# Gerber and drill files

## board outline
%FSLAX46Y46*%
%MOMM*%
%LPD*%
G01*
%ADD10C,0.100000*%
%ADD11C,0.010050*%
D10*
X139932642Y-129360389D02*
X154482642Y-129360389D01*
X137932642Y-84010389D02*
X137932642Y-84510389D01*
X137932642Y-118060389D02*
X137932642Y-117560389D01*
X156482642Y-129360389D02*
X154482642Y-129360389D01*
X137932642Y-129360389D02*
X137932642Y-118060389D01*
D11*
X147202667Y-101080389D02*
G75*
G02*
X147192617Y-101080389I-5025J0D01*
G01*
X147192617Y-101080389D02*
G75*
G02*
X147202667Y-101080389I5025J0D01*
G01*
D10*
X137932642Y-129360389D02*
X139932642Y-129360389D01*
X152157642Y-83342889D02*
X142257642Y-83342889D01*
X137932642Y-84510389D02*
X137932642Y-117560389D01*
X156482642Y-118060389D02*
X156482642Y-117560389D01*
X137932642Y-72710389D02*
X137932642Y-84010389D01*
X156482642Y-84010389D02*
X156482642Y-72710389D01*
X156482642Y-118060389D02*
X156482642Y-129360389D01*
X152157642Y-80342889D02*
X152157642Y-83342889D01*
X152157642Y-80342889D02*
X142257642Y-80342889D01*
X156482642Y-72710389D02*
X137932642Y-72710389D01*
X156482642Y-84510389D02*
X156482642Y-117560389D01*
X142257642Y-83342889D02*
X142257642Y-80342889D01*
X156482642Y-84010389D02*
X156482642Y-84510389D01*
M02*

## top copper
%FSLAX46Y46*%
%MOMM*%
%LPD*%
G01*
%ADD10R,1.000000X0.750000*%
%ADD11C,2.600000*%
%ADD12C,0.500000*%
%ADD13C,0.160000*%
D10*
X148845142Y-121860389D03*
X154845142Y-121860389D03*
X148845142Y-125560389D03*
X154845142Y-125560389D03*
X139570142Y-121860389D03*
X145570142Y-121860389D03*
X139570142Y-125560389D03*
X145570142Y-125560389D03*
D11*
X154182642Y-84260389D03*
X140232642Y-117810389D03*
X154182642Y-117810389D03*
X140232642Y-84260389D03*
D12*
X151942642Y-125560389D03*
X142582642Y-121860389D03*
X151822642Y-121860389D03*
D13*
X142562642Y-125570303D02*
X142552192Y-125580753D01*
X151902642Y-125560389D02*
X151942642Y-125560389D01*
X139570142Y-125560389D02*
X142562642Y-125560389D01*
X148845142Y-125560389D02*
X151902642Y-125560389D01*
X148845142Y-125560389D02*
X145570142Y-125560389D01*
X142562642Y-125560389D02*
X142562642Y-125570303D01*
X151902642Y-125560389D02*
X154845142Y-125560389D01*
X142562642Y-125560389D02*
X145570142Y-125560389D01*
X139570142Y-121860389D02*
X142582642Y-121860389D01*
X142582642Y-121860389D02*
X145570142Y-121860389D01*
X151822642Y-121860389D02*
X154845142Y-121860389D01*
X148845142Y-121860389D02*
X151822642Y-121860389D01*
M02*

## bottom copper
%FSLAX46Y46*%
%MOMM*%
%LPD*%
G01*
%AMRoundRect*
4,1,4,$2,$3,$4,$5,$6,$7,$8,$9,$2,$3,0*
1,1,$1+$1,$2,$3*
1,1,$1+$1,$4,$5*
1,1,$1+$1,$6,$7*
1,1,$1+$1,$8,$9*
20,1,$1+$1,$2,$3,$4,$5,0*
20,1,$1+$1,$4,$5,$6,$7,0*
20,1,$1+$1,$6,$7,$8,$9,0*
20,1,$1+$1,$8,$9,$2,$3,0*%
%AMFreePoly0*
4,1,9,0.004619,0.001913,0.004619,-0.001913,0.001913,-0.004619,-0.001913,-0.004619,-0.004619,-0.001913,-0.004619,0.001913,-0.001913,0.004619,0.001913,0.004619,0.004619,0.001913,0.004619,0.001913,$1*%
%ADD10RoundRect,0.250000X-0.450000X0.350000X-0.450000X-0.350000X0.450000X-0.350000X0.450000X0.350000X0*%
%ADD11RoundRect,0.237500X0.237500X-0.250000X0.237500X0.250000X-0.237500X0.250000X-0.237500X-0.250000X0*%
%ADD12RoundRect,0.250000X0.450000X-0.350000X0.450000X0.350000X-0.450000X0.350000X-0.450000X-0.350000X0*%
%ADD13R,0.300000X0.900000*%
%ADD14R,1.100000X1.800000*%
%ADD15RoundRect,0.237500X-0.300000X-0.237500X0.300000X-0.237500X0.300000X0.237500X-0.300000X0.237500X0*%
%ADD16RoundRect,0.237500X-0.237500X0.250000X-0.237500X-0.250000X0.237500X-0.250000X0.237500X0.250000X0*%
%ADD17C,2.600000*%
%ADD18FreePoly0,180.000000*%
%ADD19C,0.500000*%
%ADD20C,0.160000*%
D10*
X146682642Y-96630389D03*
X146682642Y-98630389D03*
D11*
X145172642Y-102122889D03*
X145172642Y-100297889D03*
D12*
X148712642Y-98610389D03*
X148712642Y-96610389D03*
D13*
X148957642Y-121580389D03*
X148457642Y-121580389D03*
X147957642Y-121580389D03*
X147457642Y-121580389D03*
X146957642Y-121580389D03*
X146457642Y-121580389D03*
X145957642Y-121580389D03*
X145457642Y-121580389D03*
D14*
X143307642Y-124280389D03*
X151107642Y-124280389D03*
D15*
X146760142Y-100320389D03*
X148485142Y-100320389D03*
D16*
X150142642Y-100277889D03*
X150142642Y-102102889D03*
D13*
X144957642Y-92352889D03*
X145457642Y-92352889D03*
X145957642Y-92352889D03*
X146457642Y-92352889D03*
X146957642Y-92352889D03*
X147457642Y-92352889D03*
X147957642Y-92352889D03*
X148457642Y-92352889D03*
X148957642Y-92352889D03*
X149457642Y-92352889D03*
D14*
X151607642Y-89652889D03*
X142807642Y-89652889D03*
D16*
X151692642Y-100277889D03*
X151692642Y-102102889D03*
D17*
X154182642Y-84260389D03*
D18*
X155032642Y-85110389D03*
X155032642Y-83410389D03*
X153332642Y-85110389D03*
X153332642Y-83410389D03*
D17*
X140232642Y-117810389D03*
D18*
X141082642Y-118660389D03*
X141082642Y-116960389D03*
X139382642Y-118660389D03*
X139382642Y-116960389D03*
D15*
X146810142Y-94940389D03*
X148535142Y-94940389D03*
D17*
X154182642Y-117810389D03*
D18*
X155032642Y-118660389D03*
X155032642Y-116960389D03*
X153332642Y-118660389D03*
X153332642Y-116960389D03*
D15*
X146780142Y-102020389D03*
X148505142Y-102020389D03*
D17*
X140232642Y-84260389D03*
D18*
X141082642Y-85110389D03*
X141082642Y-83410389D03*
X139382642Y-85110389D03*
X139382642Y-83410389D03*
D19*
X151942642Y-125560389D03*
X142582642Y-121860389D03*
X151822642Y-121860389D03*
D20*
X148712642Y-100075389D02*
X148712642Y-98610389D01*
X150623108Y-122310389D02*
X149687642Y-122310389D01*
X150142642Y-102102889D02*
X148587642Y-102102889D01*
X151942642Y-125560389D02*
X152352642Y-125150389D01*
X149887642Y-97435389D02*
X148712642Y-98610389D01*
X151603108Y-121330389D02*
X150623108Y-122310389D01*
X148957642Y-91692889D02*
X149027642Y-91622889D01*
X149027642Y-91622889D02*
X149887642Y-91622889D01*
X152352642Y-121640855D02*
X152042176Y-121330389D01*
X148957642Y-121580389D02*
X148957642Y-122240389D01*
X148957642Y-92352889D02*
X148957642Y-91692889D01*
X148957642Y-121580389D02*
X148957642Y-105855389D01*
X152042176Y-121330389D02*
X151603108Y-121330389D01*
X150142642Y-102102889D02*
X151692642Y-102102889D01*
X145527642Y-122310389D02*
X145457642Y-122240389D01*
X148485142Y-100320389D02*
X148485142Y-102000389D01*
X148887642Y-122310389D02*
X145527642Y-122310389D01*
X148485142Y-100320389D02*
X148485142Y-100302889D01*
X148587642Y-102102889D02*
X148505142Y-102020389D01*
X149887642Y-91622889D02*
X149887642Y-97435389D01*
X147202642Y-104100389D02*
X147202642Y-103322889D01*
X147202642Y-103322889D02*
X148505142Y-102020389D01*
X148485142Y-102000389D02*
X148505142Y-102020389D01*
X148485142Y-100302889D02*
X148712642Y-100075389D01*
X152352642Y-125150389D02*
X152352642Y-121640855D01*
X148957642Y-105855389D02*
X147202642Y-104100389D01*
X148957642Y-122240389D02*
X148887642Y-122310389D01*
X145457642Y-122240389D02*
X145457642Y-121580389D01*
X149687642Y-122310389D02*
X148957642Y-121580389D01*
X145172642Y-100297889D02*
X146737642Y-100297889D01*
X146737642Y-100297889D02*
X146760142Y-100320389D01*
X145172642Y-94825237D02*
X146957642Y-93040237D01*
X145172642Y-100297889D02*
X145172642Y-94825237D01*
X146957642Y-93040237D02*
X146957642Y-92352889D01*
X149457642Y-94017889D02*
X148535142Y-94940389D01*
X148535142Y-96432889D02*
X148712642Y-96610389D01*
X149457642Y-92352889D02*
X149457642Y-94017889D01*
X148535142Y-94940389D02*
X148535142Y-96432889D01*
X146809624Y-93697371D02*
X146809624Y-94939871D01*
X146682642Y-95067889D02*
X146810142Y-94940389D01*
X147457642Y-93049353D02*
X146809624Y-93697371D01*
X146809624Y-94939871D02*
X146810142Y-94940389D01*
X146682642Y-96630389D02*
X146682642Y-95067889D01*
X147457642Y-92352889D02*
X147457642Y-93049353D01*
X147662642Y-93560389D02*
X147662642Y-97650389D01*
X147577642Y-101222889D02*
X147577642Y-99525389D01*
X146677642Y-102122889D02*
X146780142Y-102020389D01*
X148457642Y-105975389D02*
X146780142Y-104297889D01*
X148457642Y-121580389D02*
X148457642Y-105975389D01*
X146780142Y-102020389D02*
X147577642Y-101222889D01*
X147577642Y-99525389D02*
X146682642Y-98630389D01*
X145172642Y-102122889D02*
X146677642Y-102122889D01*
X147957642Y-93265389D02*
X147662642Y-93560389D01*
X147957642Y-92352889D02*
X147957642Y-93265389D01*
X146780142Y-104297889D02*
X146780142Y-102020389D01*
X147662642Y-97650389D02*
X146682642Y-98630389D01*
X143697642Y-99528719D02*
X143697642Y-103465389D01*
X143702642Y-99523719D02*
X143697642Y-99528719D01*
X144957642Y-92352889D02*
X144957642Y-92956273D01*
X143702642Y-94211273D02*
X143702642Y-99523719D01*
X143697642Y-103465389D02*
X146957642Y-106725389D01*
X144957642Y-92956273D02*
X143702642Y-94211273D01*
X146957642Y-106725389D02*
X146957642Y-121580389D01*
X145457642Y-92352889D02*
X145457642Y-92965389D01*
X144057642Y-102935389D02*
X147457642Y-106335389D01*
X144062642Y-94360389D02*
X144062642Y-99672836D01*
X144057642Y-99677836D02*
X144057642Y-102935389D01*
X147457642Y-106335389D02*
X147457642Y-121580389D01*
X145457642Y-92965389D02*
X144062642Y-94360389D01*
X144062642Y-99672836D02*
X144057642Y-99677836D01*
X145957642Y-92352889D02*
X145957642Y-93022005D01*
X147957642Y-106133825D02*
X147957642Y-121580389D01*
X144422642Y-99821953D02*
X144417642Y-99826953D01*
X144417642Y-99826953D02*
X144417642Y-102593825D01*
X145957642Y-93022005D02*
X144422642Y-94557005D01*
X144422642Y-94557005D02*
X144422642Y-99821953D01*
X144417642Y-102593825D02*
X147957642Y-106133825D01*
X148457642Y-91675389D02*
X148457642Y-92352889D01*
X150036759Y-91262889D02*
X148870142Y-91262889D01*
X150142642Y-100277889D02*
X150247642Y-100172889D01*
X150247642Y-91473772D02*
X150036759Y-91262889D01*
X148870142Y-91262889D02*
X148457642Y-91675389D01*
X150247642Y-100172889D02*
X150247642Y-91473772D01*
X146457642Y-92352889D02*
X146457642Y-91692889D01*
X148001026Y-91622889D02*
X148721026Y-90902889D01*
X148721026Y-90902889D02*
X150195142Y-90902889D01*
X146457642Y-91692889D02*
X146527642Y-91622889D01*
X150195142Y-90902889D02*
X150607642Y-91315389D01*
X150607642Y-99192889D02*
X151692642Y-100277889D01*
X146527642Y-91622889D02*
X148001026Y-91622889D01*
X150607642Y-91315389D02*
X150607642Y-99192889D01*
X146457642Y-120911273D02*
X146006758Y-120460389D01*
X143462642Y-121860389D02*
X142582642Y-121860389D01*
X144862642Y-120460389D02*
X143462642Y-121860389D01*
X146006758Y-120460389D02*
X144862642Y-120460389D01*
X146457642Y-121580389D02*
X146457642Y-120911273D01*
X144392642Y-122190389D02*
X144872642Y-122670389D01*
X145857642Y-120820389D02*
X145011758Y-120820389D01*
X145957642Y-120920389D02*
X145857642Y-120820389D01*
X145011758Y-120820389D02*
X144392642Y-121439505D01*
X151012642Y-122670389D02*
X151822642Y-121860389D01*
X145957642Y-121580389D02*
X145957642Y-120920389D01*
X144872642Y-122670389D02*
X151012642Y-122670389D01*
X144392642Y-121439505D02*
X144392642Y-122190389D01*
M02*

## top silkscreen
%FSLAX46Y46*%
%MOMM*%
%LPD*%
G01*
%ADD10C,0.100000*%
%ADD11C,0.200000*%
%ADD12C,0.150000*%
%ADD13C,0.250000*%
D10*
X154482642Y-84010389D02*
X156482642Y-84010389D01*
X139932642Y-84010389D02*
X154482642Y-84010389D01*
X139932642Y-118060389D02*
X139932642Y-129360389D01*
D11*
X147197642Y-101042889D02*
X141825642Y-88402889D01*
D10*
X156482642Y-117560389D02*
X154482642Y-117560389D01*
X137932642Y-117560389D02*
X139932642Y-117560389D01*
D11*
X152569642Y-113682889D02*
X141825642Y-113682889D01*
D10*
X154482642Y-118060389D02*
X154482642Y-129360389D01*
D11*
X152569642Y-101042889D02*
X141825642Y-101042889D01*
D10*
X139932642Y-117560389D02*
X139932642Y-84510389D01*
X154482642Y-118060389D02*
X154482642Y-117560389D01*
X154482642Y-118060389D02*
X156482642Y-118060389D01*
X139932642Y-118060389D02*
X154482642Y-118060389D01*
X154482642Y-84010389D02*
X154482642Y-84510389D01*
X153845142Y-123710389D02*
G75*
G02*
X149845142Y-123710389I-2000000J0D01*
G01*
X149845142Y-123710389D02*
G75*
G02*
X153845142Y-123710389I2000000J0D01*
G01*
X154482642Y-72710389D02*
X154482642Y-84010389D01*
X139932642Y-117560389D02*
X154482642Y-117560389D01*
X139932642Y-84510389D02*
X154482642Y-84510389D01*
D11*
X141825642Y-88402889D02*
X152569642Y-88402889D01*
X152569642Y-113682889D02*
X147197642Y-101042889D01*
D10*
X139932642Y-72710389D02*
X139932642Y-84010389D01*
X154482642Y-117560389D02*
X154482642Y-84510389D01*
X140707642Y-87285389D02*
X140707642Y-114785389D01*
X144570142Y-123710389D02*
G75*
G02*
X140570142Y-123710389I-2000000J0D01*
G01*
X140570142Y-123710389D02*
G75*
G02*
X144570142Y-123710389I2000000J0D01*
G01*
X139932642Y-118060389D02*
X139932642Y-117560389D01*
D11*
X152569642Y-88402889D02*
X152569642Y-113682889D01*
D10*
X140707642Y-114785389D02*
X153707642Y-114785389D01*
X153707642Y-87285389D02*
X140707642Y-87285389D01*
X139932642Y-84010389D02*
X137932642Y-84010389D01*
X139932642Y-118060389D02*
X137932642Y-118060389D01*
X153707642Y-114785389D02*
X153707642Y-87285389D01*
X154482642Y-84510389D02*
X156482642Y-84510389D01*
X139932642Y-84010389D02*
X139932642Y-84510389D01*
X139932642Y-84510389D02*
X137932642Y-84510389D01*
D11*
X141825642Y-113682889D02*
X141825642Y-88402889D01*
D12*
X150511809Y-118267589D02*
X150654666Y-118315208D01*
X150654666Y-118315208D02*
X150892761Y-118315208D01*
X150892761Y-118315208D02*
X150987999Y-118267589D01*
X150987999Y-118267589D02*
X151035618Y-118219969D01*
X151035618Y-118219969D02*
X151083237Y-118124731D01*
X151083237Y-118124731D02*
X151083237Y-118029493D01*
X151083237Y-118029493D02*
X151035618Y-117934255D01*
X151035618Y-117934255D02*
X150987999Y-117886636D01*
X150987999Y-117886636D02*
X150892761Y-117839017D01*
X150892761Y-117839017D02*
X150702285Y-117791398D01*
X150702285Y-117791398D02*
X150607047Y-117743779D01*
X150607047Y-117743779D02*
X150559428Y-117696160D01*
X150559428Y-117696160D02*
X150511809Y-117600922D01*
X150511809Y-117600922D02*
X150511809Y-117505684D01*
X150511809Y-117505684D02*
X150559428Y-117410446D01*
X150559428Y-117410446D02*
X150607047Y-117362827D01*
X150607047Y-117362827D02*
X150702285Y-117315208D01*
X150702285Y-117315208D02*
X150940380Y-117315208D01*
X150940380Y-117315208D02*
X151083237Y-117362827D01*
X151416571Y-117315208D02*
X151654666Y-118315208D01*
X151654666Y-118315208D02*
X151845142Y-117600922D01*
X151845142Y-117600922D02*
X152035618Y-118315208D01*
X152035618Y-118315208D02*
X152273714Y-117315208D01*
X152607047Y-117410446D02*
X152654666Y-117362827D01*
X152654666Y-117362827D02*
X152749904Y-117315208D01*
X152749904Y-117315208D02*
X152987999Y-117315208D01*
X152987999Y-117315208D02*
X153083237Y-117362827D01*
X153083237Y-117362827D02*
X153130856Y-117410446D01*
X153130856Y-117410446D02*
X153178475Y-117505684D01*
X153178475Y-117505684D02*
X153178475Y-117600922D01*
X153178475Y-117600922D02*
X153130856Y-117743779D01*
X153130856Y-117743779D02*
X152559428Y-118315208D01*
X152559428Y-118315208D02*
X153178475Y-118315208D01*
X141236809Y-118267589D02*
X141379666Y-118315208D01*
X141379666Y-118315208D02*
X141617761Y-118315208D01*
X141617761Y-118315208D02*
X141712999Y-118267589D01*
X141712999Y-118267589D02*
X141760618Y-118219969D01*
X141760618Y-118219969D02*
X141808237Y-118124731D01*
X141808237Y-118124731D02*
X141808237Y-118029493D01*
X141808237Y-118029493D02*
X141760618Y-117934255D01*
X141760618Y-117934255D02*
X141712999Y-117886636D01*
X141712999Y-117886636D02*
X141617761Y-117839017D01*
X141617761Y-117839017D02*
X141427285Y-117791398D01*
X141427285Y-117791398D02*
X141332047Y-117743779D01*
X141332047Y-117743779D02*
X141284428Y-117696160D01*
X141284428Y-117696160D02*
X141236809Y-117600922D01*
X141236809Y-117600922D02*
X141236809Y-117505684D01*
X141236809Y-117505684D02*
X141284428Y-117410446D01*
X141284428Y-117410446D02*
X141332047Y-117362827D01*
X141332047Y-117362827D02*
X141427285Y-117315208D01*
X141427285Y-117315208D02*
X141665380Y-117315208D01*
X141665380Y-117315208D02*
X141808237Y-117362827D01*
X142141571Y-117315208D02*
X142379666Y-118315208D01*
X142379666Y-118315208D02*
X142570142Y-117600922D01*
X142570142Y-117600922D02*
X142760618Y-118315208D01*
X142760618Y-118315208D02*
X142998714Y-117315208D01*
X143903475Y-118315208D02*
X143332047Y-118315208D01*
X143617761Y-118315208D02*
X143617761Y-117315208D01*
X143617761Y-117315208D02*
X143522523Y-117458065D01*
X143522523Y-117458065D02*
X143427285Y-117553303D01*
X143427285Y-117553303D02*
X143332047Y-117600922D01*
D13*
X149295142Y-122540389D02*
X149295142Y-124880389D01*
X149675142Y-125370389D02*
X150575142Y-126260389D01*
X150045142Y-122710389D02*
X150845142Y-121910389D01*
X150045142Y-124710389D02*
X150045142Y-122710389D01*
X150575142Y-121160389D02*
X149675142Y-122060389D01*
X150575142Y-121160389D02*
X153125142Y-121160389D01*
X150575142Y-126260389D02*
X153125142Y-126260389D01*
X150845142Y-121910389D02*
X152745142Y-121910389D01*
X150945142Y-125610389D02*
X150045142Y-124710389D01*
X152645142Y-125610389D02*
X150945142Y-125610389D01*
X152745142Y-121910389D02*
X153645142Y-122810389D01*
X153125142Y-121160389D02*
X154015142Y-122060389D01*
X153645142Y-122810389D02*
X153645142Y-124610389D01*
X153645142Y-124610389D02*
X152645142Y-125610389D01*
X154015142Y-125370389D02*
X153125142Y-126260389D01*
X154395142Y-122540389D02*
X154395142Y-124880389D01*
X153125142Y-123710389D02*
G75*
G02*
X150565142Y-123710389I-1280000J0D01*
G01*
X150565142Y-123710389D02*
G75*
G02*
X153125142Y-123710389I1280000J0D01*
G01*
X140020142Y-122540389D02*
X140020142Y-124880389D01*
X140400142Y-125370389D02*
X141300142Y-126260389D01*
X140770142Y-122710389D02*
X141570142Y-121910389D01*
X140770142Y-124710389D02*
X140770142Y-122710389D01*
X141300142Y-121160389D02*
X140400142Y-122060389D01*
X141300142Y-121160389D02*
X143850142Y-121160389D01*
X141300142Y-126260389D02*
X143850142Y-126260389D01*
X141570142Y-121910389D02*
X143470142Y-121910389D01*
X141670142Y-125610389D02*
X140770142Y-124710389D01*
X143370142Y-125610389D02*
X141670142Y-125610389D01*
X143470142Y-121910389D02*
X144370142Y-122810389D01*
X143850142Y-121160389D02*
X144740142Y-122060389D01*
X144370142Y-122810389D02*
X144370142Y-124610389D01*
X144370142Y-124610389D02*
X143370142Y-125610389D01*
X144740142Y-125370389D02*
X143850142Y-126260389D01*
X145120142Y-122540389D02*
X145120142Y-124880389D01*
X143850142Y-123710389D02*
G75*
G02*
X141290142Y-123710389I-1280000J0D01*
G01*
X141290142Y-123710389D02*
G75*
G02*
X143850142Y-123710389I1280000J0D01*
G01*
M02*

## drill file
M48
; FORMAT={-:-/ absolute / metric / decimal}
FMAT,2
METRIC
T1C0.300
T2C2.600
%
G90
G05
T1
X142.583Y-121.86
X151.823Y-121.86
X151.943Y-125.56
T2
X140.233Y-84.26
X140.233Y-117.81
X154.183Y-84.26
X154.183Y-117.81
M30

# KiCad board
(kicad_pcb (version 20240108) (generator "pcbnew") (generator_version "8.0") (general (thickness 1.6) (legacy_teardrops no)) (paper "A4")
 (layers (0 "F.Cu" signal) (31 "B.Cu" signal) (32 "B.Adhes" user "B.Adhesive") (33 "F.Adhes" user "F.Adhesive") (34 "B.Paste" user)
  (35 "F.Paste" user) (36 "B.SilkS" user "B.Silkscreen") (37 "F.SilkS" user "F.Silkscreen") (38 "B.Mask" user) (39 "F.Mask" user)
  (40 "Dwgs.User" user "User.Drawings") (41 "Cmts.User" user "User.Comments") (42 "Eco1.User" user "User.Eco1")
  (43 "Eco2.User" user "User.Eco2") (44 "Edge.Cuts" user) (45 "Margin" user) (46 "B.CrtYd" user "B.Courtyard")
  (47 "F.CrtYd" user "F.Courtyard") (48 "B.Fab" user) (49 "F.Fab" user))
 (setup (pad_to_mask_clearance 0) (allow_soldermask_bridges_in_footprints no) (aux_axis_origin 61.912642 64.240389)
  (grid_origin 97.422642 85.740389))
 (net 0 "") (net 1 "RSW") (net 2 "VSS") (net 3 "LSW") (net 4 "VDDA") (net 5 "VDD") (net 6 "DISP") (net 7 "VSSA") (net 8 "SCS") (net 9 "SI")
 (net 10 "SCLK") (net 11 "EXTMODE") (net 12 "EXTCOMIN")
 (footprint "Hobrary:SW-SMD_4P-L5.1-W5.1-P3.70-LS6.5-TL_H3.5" (layer "F.Cu") (at 151.845142 123.710389)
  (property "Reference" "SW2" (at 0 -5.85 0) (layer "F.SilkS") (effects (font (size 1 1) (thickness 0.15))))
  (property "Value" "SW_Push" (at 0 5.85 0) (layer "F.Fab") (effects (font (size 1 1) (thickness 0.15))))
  (fp_line (start -2.55 -1.17) (end -2.55 1.17) (stroke (width 0.25) (type solid)) (layer "F.SilkS"))
  (fp_line (start -2.17 1.66) (end -1.27 2.55) (stroke (width 0.25) (type solid)) (layer "F.SilkS"))
  (fp_line (start -1.8 -1) (end -1 -1.8) (stroke (width 0.25) (type solid)) (layer "F.SilkS"))
  (fp_line (start -1.8 1) (end -1.8 -1) (stroke (width 0.25) (type solid)) (layer "F.SilkS"))
  (fp_line (start -1.27 -2.55) (end -2.17 -1.65) (stroke (width 0.25) (type solid)) (layer "F.SilkS"))
  (fp_line (start -1.27 -2.55) (end 1.28 -2.55) (stroke (width 0.25) (type solid)) (layer "F.SilkS"))
  (fp_line (start -1.27 2.55) (end 1.28 2.55) (stroke (width 0.25) (type solid)) (layer "F.SilkS"))
  (fp_line (start -1 -1.8) (end 0.9 -1.8) (stroke (width 0.25) (type solid)) (layer "F.SilkS"))
  (fp_line (start -0.9 1.9) (end -1.8 1) (stroke (width 0.25) (type solid)) (layer "F.SilkS"))
  (fp_line (start 0.8 1.9) (end -0.9 1.9) (stroke (width 0.25) (type solid)) (layer "F.SilkS"))
  (fp_line (start 0.9 -1.8) (end 1.8 -0.9) (stroke (width 0.25) (type solid)) (layer "F.SilkS"))
  (fp_line (start 1.28 -2.55) (end 2.17 -1.65) (stroke (width 0.25) (type solid)) (layer "F.SilkS"))
  (fp_line (start 1.8 -0.9) (end 1.8 0.9) (stroke (width 0.25) (type solid)) (layer "F.SilkS"))
  (fp_line (start 1.8 0.9) (end 0.8 1.9) (stroke (width 0.25) (type solid)) (layer "F.SilkS"))
  (fp_line (start 2.17 1.66) (end 1.28 2.55) (stroke (width 0.25) (type solid)) (layer "F.SilkS"))
  (fp_line (start 2.55 -1.17) (end 2.55 1.17) (stroke (width 0.25) (type solid)) (layer "F.SilkS"))
  (fp_circle (center 0 0) (end 1.28 0) (stroke (width 0.25) (type solid)) (fill none) (layer "F.SilkS"))
  (pad "1" smd rect (at -3 -1.85) (size 1 0.75) (layers "F.Cu" "F.Paste" "F.Mask") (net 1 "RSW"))
  (pad "1" smd rect (at 3 -1.85) (size 1 0.75) (layers "F.Cu" "F.Paste" "F.Mask") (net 1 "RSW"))
  (pad "2" smd rect (at -3 1.85) (size 1 0.75) (layers "F.Cu" "F.Paste" "F.Mask") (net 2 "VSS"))
  (pad "2" smd rect (at 3 1.85) (size 1 0.75) (layers "F.Cu" "F.Paste" "F.Mask") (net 2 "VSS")))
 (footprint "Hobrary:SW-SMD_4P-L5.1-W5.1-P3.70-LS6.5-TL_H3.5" (layer "F.Cu") (at 142.570142 123.710389)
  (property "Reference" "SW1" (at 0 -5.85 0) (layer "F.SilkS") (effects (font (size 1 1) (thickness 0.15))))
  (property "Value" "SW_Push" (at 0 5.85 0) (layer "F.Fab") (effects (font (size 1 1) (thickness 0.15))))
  (fp_line (start -2.55 -1.17) (end -2.55 1.17) (stroke (width 0.25) (type solid)) (layer "F.SilkS"))
  (fp_line (start -2.17 1.66) (end -1.27 2.55) (stroke (width 0.25) (type solid)) (layer "F.SilkS"))
  (fp_line (start -1.8 -1) (end -1 -1.8) (stroke (width 0.25) (type solid)) (layer "F.SilkS"))
  (fp_line (start -1.8 1) (end -1.8 -1) (stroke (width 0.25) (type solid)) (layer "F.SilkS"))
  (fp_line (start -1.27 -2.55) (end -2.17 -1.65) (stroke (width 0.25) (type solid)) (layer "F.SilkS"))
  (fp_line (start -1.27 -2.55) (end 1.28 -2.55) (stroke (width 0.25) (type solid)) (layer "F.SilkS"))
  (fp_line (start -1.27 2.55) (end 1.28 2.55) (stroke (width 0.25) (type solid)) (layer "F.SilkS"))
  (fp_line (start -1 -1.8) (end 0.9 -1.8) (stroke (width 0.25) (type solid)) (layer "F.SilkS"))
  (fp_line (start -0.9 1.9) (end -1.8 1) (stroke (width 0.25) (type solid)) (layer "F.SilkS"))
  (fp_line (start 0.8 1.9) (end -0.9 1.9) (stroke (width 0.25) (type solid)) (layer "F.SilkS"))
  (fp_line (start 0.9 -1.8) (end 1.8 -0.9) (stroke (width 0.25) (type solid)) (layer "F.SilkS"))
  (fp_line (start 1.28 -2.55) (end 2.17 -1.65) (stroke (width 0.25) (type solid)) (layer "F.SilkS"))
  (fp_line (start 1.8 -0.9) (end 1.8 0.9) (stroke (width 0.25) (type solid)) (layer "F.SilkS"))
  (fp_line (start 1.8 0.9) (end 0.8 1.9) (stroke (width 0.25) (type solid)) (layer "F.SilkS"))
  (fp_line (start 2.17 1.66) (end 1.28 2.55) (stroke (width 0.25) (type solid)) (layer "F.SilkS"))
  (fp_line (start 2.55 -1.17) (end 2.55 1.17) (stroke (width 0.25) (type solid)) (layer "F.SilkS"))
  (fp_circle (center 0 0) (end 1.28 0) (stroke (width 0.25) (type solid)) (fill none) (layer "F.SilkS"))
  (pad "1" smd rect (at -3 -1.85) (size 1 0.75) (layers "F.Cu" "F.Paste" "F.Mask") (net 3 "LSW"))
  (pad "1" smd rect (at 3 -1.85) (size 1 0.75) (layers "F.Cu" "F.Paste" "F.Mask") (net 3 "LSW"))
  (pad "2" smd rect (at -3 1.85) (size 1 0.75) (layers "F.Cu" "F.Paste" "F.Mask") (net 2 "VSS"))
  (pad "2" smd rect (at 3 1.85) (size 1 0.75) (layers "F.Cu" "F.Paste" "F.Mask") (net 2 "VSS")))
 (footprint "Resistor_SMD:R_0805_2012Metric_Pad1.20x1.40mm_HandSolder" (layer "B.Cu") (at 146.682642 97.630389 -90)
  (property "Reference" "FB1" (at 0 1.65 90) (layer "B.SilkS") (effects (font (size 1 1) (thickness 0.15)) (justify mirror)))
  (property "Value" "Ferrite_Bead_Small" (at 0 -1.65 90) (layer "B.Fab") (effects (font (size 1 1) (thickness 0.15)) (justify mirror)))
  (pad "1" smd roundrect (at -1 0 270) (size 1.2 1.4) (layers "B.Cu" "B.Paste" "B.Mask") (roundrect_rratio 0.208333) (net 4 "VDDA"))
  (pad "2" smd roundrect (at 1 0 270) (size 1.2 1.4) (layers "B.Cu" "B.Paste" "B.Mask") (roundrect_rratio 0.208333) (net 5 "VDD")))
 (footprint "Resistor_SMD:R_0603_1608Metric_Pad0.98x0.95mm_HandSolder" (layer "B.Cu") (at 145.172642 101.210389 90)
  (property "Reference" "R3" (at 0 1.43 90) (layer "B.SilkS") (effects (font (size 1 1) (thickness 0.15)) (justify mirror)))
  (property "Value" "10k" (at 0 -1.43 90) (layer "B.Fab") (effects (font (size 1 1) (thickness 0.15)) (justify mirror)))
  (pad "1" smd roundrect (at -0.9125 0 90) (size 0.975 0.95) (layers "B.Cu" "B.Paste" "B.Mask") (roundrect_rratio 0.25) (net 5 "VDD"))
  (pad "2" smd roundrect (at 0.9125 0 90) (size 0.975 0.95) (layers "B.Cu" "B.Paste" "B.Mask") (roundrect_rratio 0.25) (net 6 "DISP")))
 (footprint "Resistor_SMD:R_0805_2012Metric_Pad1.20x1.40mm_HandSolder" (layer "B.Cu") (at 148.712642 97.610389 90)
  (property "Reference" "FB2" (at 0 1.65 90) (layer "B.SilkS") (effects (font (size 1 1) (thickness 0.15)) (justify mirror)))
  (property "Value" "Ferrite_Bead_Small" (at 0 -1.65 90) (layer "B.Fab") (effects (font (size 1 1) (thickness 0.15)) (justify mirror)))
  (pad "1" smd roundrect (at -1 0 90) (size 1.2 1.4) (layers "B.Cu" "B.Paste" "B.Mask") (roundrect_rratio 0.208333) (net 2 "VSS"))
  (pad "2" smd roundrect (at 1 0 90) (size 1.2 1.4) (layers "B.Cu" "B.Paste" "B.Mask") (roundrect_rratio 0.208333) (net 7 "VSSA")))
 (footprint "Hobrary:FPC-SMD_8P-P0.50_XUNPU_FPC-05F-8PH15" (layer "B.Cu") (at 147.207642 122.930389 180)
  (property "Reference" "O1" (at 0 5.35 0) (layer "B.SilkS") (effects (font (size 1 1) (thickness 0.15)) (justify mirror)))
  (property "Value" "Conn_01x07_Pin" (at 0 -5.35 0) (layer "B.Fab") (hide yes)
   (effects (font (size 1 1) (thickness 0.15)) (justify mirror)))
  (pad "1" smd rect (at -1.75 1.35 180) (size 0.3 0.9) (layers "B.Cu" "B.Paste" "B.Mask") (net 2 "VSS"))
  (pad "2" smd rect (at -1.25 1.35 180) (size 0.3 0.9) (layers "B.Cu" "B.Paste" "B.Mask") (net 5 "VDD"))
  (pad "3" smd rect (at -0.75 1.35 180) (size 0.3 0.9) (layers "B.Cu" "B.Paste" "B.Mask") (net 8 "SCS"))
  (pad "4" smd rect (at -0.25 1.35 180) (size 0.3 0.9) (layers "B.Cu" "B.Paste" "B.Mask") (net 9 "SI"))
  (pad "5" smd rect (at 0.25 1.35 180) (size 0.3 0.9) (layers "B.Cu" "B.Paste" "B.Mask") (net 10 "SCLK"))
  (pad "6" smd rect (at 0.75 1.35 180) (size 0.3 0.9) (layers "B.Cu" "B.Paste" "B.Mask") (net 3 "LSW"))
  (pad "7" smd rect (at 1.25 1.35 180) (size 0.3 0.9) (layers "B.Cu" "B.Paste" "B.Mask") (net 1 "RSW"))
  (pad "8" smd rect (at 1.75 1.35 180) (size 0.3 0.9) (layers "B.Cu" "B.Paste" "B.Mask") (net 2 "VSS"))
  (pad "9" smd rect (at 3.9 -1.35 180) (size 1.1 1.8) (layers "B.Cu" "B.Paste" "B.Mask"))
  (pad "10" smd rect (at -3.9 -1.35 180) (size 1.1 1.8) (layers "B.Cu" "B.Paste" "B.Mask")))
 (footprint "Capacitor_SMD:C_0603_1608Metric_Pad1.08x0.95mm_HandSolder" (layer "B.Cu") (at 147.622642 100.320389)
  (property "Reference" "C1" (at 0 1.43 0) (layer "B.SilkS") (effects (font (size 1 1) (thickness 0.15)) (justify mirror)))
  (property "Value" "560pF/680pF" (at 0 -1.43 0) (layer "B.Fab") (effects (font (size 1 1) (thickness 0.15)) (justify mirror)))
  (pad "1" smd roundrect (at -0.8625 0) (size 1.075 0.95) (layers "B.Cu" "B.Paste" "B.Mask") (roundrect_rratio 0.25) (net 6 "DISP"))
  (pad "2" smd roundrect (at 0.8625 0) (size 1.075 0.95) (layers "B.Cu" "B.Paste" "B.Mask") (roundrect_rratio 0.25) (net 2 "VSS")))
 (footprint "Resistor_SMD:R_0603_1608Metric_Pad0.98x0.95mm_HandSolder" (layer "B.Cu") (at 150.142642 101.190389 -90)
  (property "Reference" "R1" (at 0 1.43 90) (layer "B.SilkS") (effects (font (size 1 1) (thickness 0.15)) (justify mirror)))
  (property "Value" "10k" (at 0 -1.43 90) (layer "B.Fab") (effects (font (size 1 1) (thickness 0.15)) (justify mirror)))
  (pad "1" smd roundrect (at -0.9125 0 270) (size 0.975 0.95) (layers "B.Cu" "B.Paste" "B.Mask") (roundrect_rratio 0.25) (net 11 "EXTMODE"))
  (pad "2" smd roundrect (at 0.9125 0 270) (size 0.975 0.95) (layers "B.Cu" "B.Paste" "B.Mask") (roundrect_rratio 0.25) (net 2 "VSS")))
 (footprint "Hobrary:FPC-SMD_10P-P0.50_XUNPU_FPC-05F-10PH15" (layer "B.Cu") (at 147.207642 91.002889)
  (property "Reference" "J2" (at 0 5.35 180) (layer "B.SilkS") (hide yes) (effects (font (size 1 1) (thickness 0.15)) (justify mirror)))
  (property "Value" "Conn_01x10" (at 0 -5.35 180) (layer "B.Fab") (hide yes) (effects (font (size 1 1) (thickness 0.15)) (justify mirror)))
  (pad "1" smd rect (at -2.25 1.35) (size 0.3 0.9) (layers "B.Cu" "B.Paste" "B.Mask") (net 10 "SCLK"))
  (pad "2" smd rect (at -1.75 1.35) (size 0.3 0.9) (layers "B.Cu" "B.Paste" "B.Mask") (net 9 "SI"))
  (pad "3" smd rect (at -1.25 1.35) (size 0.3 0.9) (layers "B.Cu" "B.Paste" "B.Mask") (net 8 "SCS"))
  (pad "4" smd rect (at -0.75 1.35) (size 0.3 0.9) (layers "B.Cu" "B.Paste" "B.Mask") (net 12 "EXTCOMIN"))
  (pad "5" smd rect (at -0.25 1.35) (size 0.3 0.9) (layers "B.Cu" "B.Paste" "B.Mask") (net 6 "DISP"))
  (pad "6" smd rect (at 0.25 1.35) (size 0.3 0.9) (layers "B.Cu" "B.Paste" "B.Mask") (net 4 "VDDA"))
  (pad "7" smd rect (at 0.75 1.35) (size 0.3 0.9) (layers "B.Cu" "B.Paste" "B.Mask") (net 5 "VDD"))
  (pad "8" smd rect (at 1.25 1.35) (size 0.3 0.9) (layers "B.Cu" "B.Paste" "B.Mask") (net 11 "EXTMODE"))
  (pad "9" smd rect (at 1.75 1.35) (size 0.3 0.9) (layers "B.Cu" "B.Paste" "B.Mask") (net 2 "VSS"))
  (pad "10" smd rect (at 2.25 1.35) (size 0.3 0.9) (layers "B.Cu" "B.Paste" "B.Mask") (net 7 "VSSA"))
  (pad "11" smd rect (at 4.4 -1.35) (size 1.1 1.8) (layers "B.Cu" "B.Paste" "B.Mask"))
  (pad "12" smd rect (at -4.4 -1.35) (size 1.1 1.8) (layers "B.Cu" "B.Paste" "B.Mask")))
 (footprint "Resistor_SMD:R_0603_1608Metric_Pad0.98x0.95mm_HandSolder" (layer "B.Cu") (at 151.692642 101.190389 -90)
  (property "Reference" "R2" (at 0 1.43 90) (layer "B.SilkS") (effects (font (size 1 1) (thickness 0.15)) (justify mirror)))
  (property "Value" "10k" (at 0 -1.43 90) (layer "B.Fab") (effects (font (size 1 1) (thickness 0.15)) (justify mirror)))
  (pad "1" smd roundrect (at -0.9125 0 270) (size 0.975 0.95) (layers "B.Cu" "B.Paste" "B.Mask") (roundrect_rratio 0.25) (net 12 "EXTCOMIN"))
  (pad "2" smd roundrect (at 0.9125 0 270) (size 0.975 0.95) (layers "B.Cu" "B.Paste" "B.Mask") (roundrect_rratio 0.25) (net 2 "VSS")))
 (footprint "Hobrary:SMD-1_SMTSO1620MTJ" (layer "B.Cu") (at 154.182642 84.260389 180)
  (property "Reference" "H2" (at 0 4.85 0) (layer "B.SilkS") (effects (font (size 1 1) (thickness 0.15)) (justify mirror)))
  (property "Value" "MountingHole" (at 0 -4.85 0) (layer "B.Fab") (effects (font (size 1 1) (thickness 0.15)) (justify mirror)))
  (pad "" thru_hole circle (at 0 0 180) (size 2.6 2.6) (drill 2.6) (layers "*.Cu" "*.Mask") (remove_unused_layers no))
  (pad "1" smd custom (at -0.85 -0.85 180) (size 0.01 0.01) (layers "B.Cu" "B.Paste" "B.Mask") (thermal_bridge_angle 90)
   (options (clearance outline) (anchor circle)) (primitives))
  (pad "1" smd custom (at -0.85 0.85 180) (size 0.01 0.01) (layers "B.Cu" "B.Paste" "B.Mask") (thermal_bridge_angle 90)
   (options (clearance outline) (anchor circle)) (primitives))
  (pad "1" smd custom (at 0.85 -0.85 180) (size 0.01 0.01) (layers "B.Cu" "B.Paste" "B.Mask") (thermal_bridge_angle 90)
   (options (clearance outline) (anchor circle)) (primitives))
  (pad "1" smd custom (at 0.85 0.85 180) (size 0.01 0.01) (layers "B.Cu" "B.Paste" "B.Mask") (thermal_bridge_angle 90)
   (options (clearance outline) (anchor circle)) (primitives)))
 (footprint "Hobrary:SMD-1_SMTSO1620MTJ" (layer "B.Cu") (at 140.232642 117.810389 180)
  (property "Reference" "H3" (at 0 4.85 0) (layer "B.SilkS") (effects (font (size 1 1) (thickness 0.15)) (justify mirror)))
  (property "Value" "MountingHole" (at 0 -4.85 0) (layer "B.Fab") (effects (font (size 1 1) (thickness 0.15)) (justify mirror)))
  (pad "" thru_hole circle (at 0 0 180) (size 2.6 2.6) (drill 2.6) (layers "*.Cu" "*.Mask") (remove_unused_layers no))
  (pad "1" smd custom (at -0.85 -0.85 180) (size 0.01 0.01) (layers "B.Cu" "B.Paste" "B.Mask") (thermal_bridge_angle 90)
   (options (clearance outline) (anchor circle)) (primitives))
  (pad "1" smd custom (at -0.85 0.85 180) (size 0.01 0.01) (layers "B.Cu" "B.Paste" "B.Mask") (thermal_bridge_angle 90)
   (options (clearance outline) (anchor circle)) (primitives))
  (pad "1" smd custom (at 0.85 -0.85 180) (size 0.01 0.01) (layers "B.Cu" "B.Paste" "B.Mask") (thermal_bridge_angle 90)
   (options (clearance outline) (anchor circle)) (primitives))
  (pad "1" smd custom (at 0.85 0.85 180) (size 0.01 0.01) (layers "B.Cu" "B.Paste" "B.Mask") (thermal_bridge_angle 90)
   (options (clearance outline) (anchor circle)) (primitives)))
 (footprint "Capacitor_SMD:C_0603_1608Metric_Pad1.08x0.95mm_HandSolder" (layer "B.Cu") (at 147.672642 94.940389)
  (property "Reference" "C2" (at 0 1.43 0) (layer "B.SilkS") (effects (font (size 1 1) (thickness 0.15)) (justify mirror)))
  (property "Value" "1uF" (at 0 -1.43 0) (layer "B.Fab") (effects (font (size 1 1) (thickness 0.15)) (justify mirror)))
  (pad "1" smd roundrect (at -0.8625 0) (size 1.075 0.95) (layers "B.Cu" "B.Paste" "B.Mask") (roundrect_rratio 0.25) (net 4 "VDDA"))
  (pad "2" smd roundrect (at 0.8625 0) (size 1.075 0.95) (layers "B.Cu" "B.Paste" "B.Mask") (roundrect_rratio 0.25) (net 7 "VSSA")))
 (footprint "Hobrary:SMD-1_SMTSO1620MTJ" (layer "B.Cu") (at 154.182642 117.810389 180)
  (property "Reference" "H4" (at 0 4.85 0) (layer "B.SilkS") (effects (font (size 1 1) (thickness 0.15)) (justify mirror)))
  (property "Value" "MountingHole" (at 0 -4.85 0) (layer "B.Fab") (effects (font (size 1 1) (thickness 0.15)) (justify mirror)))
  (pad "" thru_hole circle (at 0 0 180) (size 2.6 2.6) (drill 2.6) (layers "*.Cu" "*.Mask") (remove_unused_layers no))
  (pad "1" smd custom (at -0.85 -0.85 180) (size 0.01 0.01) (layers "B.Cu" "B.Paste" "B.Mask") (thermal_bridge_angle 90)
   (options (clearance outline) (anchor circle)) (primitives))
  (pad "1" smd custom (at -0.85 0.85 180) (size 0.01 0.01) (layers "B.Cu" "B.Paste" "B.Mask") (thermal_bridge_angle 90)
   (options (clearance outline) (anchor circle)) (primitives))
  (pad "1" smd custom (at 0.85 -0.85 180) (size 0.01 0.01) (layers "B.Cu" "B.Paste" "B.Mask") (thermal_bridge_angle 90)
   (options (clearance outline) (anchor circle)) (primitives))
  (pad "1" smd custom (at 0.85 0.85 180) (size 0.01 0.01) (layers "B.Cu" "B.Paste" "B.Mask") (thermal_bridge_angle 90)
   (options (clearance outline) (anchor circle)) (primitives)))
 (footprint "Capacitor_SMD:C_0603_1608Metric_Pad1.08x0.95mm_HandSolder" (layer "B.Cu") (at 147.642642 102.020389)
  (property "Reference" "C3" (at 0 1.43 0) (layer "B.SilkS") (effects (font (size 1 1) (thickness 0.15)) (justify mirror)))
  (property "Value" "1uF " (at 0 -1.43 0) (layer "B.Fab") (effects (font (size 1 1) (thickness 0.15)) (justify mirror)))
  (pad "1" smd roundrect (at -0.8625 0) (size 1.075 0.95) (layers "B.Cu" "B.Paste" "B.Mask") (roundrect_rratio 0.25) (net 5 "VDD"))
  (pad "2" smd roundrect (at 0.8625 0) (size 1.075 0.95) (layers "B.Cu" "B.Paste" "B.Mask") (roundrect_rratio 0.25) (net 2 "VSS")))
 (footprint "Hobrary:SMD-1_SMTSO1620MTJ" (layer "B.Cu") (at 140.232642 84.260389 180)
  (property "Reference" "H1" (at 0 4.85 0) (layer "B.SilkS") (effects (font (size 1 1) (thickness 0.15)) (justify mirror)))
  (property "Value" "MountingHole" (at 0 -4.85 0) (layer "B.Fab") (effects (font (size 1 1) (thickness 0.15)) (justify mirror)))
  (pad "" thru_hole circle (at 0 0 180) (size 2.6 2.6) (drill 2.6) (layers "*.Cu" "*.Mask") (remove_unused_layers no))
  (pad "1" smd custom (at -0.85 -0.85 180) (size 0.01 0.01) (layers "B.Cu" "B.Paste" "B.Mask") (thermal_bridge_angle 90)
   (options (clearance outline) (anchor circle)) (primitives))
  (pad "1" smd custom (at -0.85 0.85 180) (size 0.01 0.01) (layers "B.Cu" "B.Paste" "B.Mask") (thermal_bridge_angle 90)
   (options (clearance outline) (anchor circle)) (primitives))
  (pad "1" smd custom (at 0.85 -0.85 180) (size 0.01 0.01) (layers "B.Cu" "B.Paste" "B.Mask") (thermal_bridge_angle 90)
   (options (clearance outline) (anchor circle)) (primitives))
  (pad "1" smd custom (at 0.85 0.85 180) (size 0.01 0.01) (layers "B.Cu" "B.Paste" "B.Mask") (thermal_bridge_angle 90)
   (options (clearance outline) (anchor circle)) (primitives)))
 (gr_line (start 154.482642 84.010389) (end 156.482642 84.010389) (stroke (width 0.1) (type default)) (layer "F.SilkS"))
 (gr_line (start 139.932642 84.010389) (end 154.482642 84.010389) (stroke (width 0.1) (type default)) (layer "F.SilkS"))
 (gr_line (start 139.932642 118.060389) (end 139.932642 129.360389) (stroke (width 0.1) (type default)) (layer "F.SilkS"))
 (gr_line (start 147.197642 101.042889) (end 141.825642 88.402889) (stroke (width 0.2) (type solid)) (layer "F.SilkS"))
 (gr_line (start 156.482642 117.560389) (end 154.482642 117.560389) (stroke (width 0.1) (type default)) (layer "F.SilkS"))
 (gr_line (start 137.932642 117.560389) (end 139.932642 117.560389) (stroke (width 0.1) (type default)) (layer "F.SilkS"))
 (gr_line (start 152.569642 113.682889) (end 141.825642 113.682889) (stroke (width 0.2) (type solid)) (layer "F.SilkS"))
 (gr_line (start 154.482642 118.060389) (end 154.482642 129.360389) (stroke (width 0.1) (type default)) (layer "F.SilkS"))
 (gr_line (start 152.569642 101.042889) (end 141.825642 101.042889) (stroke (width 0.2) (type solid)) (layer "F.SilkS"))
 (gr_line (start 139.932642 117.560389) (end 139.932642 84.510389) (stroke (width 0.1) (type default)) (layer "F.SilkS"))
 (gr_line (start 154.482642 118.060389) (end 154.482642 117.560389) (stroke (width 0.1) (type default)) (layer "F.SilkS"))
 (gr_line (start 154.482642 118.060389) (end 156.482642 118.060389) (stroke (width 0.1) (type default)) (layer "F.SilkS"))
 (gr_line (start 139.932642 118.060389) (end 154.482642 118.060389) (stroke (width 0.1) (type default)) (layer "F.SilkS"))
 (gr_line (start 154.482642 84.010389) (end 154.482642 84.510389) (stroke (width 0.1) (type default)) (layer "F.SilkS"))
 (gr_circle (center 151.845142 123.710389) (end 153.845142 123.710389) (stroke (width 0.1) (type default)) (fill none) (layer "F.SilkS"))
 (gr_line (start 154.482642 72.710389) (end 154.482642 84.010389) (stroke (width 0.1) (type default)) (layer "F.SilkS"))
 (gr_line (start 139.932642 117.560389) (end 154.482642 117.560389) (stroke (width 0.1) (type default)) (layer "F.SilkS"))
 (gr_line (start 139.932642 84.510389) (end 154.482642 84.510389) (stroke (width 0.1) (type default)) (layer "F.SilkS"))
 (gr_line (start 141.825642 88.402889) (end 152.569642 88.402889) (stroke (width 0.2) (type solid)) (layer "F.SilkS"))
 (gr_line (start 152.569642 113.682889) (end 147.197642 101.042889) (stroke (width 0.2) (type solid)) (layer "F.SilkS"))
 (gr_line (start 139.932642 72.710389) (end 139.932642 84.010389) (stroke (width 0.1) (type default)) (layer "F.SilkS"))
 (gr_line (start 154.482642 117.560389) (end 154.482642 84.510389) (stroke (width 0.1) (type default)) (layer "F.SilkS"))
 (gr_line (start 140.707642 87.285389) (end 140.707642 114.785389) (stroke (width 0.1) (type default)) (layer "F.SilkS"))
 (gr_circle (center 142.570142 123.710389) (end 144.570142 123.710389) (stroke (width 0.1) (type default)) (fill none) (layer "F.SilkS"))
 (gr_line (start 139.932642 118.060389) (end 139.932642 117.560389) (stroke (width 0.1) (type default)) (layer "F.SilkS"))
 (gr_line (start 152.569642 88.402889) (end 152.569642 113.682889) (stroke (width 0.2) (type solid)) (layer "F.SilkS"))
 (gr_line (start 140.707642 114.785389) (end 153.707642 114.785389) (stroke (width 0.1) (type default)) (layer "F.SilkS"))
 (gr_line (start 153.707642 87.285389) (end 140.707642 87.285389) (stroke (width 0.1) (type default)) (layer "F.SilkS"))
 (gr_line (start 139.932642 84.010389) (end 137.932642 84.010389) (stroke (width 0.1) (type default)) (layer "F.SilkS"))
 (gr_line (start 139.932642 118.060389) (end 137.932642 118.060389) (stroke (width 0.1) (type default)) (layer "F.SilkS"))
 (gr_line (start 153.707642 114.785389) (end 153.707642 87.285389) (stroke (width 0.1) (type default)) (layer "F.SilkS"))
 (gr_line (start 154.482642 84.510389) (end 156.482642 84.510389) (stroke (width 0.1) (type default)) (layer "F.SilkS"))
 (gr_line (start 139.932642 84.010389) (end 139.932642 84.510389) (stroke (width 0.1) (type default)) (layer "F.SilkS"))
 (gr_line (start 139.932642 84.510389) (end 137.932642 84.510389) (stroke (width 0.1) (type default)) (layer "F.SilkS"))
 (gr_line (start 141.825642 113.682889) (end 141.825642 88.402889) (stroke (width 0.2) (type solid)) (layer "F.SilkS"))
 (gr_line (start 139.932642 129.360389) (end 154.482642 129.360389) (stroke (width 0.1) (type default)) (layer "Edge.Cuts"))
 (gr_line (start 137.932642 84.010389) (end 137.932642 84.510389) (stroke (width 0.1) (type default)) (layer "Edge.Cuts"))
 (gr_line (start 137.932642 118.060389) (end 137.932642 117.560389) (stroke (width 0.1) (type default)) (layer "Edge.Cuts"))
 (gr_line (start 156.482642 129.360389) (end 154.482642 129.360389) (stroke (width 0.1) (type default)) (layer "Edge.Cuts"))
 (gr_line (start 137.932642 129.360389) (end 137.932642 118.060389) (stroke (width 0.1) (type default)) (layer "Edge.Cuts"))
 (gr_circle (center 147.197642 101.080389) (end 147.207642 101.080389) (stroke (width 0.0001) (type default)) (fill solid)
  (layer "Edge.Cuts"))
 (gr_line (start 137.932642 129.360389) (end 139.932642 129.360389) (stroke (width 0.1) (type default)) (layer "Edge.Cuts"))
 (gr_line (start 152.157642 83.342889) (end 142.257642 83.342889) (stroke (width 0.1) (type default)) (layer "Edge.Cuts"))
 (gr_line (start 137.932642 84.510389) (end 137.932642 117.560389) (stroke (width 0.1) (type default)) (layer "Edge.Cuts"))
 (gr_line (start 156.482642 118.060389) (end 156.482642 117.560389) (stroke (width 0.1) (type default)) (layer "Edge.Cuts"))
 (gr_line (start 137.932642 72.710389) (end 137.932642 84.010389) (stroke (width 0.1) (type default)) (layer "Edge.Cuts"))
 (gr_line (start 156.482642 84.010389) (end 156.482642 72.710389) (stroke (width 0.1) (type default)) (layer "Edge.Cuts"))
 (gr_line (start 156.482642 118.060389) (end 156.482642 129.360389) (stroke (width 0.1) (type default)) (layer "Edge.Cuts"))
 (gr_line (start 152.157642 80.342889) (end 152.157642 83.342889) (stroke (width 0.1) (type default)) (layer "Edge.Cuts"))
 (gr_line (start 152.157642 80.342889) (end 142.257642 80.342889) (stroke (width 0.1) (type default)) (layer "Edge.Cuts"))
 (gr_line (start 156.482642 72.710389) (end 137.932642 72.710389) (stroke (width 0.1) (type default)) (layer "Edge.Cuts"))
 (gr_line (start 156.482642 84.510389) (end 156.482642 117.560389) (stroke (width 0.1) (type default)) (layer "Edge.Cuts"))
 (gr_line (start 142.257642 83.342889) (end 142.257642 80.342889) (stroke (width 0.1) (type default)) (layer "Edge.Cuts"))
 (gr_line (start 156.482642 84.010389) (end 156.482642 84.510389) (stroke (width 0.1) (type default)) (layer "Edge.Cuts"))
 (segment (start 142.562642 125.570303) (end 142.552192 125.580753) (width 0.16) (layer "F.Cu") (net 2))
 (segment (start 151.902642 125.560389) (end 151.942642 125.560389) (width 0.16) (layer "F.Cu") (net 2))
 (segment (start 139.570142 125.560389) (end 142.562642 125.560389) (width 0.16) (layer "F.Cu") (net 2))
 (segment (start 148.845142 125.560389) (end 151.902642 125.560389) (width 0.16) (layer "F.Cu") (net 2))
 (segment (start 148.845142 125.560389) (end 145.570142 125.560389) (width 0.16) (layer "F.Cu") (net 2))
 (segment (start 142.562642 125.560389) (end 142.562642 125.570303) (width 0.16) (layer "F.Cu") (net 2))
 (segment (start 151.902642 125.560389) (end 154.845142 125.560389) (width 0.16) (layer "F.Cu") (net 2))
 (segment (start 142.562642 125.560389) (end 145.570142 125.560389) (width 0.16) (layer "F.Cu") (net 2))
 (via (at 151.942642 125.560389) (size 0.5) (drill 0.3) (layers "F.Cu" "B.Cu") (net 2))
 (segment (start 148.712642 100.075389) (end 148.712642 98.610389) (width 0.16) (layer "B.Cu") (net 2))
 (segment (start 150.623108 122.310389) (end 149.687642 122.310389) (width 0.16) (layer "B.Cu") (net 2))
 (segment (start 150.142642 102.102889) (end 148.587642 102.102889) (width 0.16) (layer "B.Cu") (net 2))
 (segment (start 151.942642 125.560389) (end 152.352642 125.150389) (width 0.16) (layer "B.Cu") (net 2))
 (segment (start 149.887642 97.435389) (end 148.712642 98.610389) (width 0.16) (layer "B.Cu") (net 2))
 (segment (start 151.603108 121.330389) (end 150.623108 122.310389) (width 0.16) (layer "B.Cu") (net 2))
 (segment (start 148.957642 91.692889) (end 149.027642 91.622889) (width 0.16) (layer "B.Cu") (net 2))
 (segment (start 149.027642 91.622889) (end 149.887642 91.622889) (width 0.16) (layer "B.Cu") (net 2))
 (segment (start 152.352642 121.640855) (end 152.042176 121.330389) (width 0.16) (layer "B.Cu") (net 2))
 (segment (start 148.957642 121.580389) (end 148.957642 122.240389) (width 0.16) (layer "B.Cu") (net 2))
 (segment (start 148.957642 92.352889) (end 148.957642 91.692889) (width 0.16) (layer "B.Cu") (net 2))
 (segment (start 148.957642 121.580389) (end 148.957642 105.855389) (width 0.16) (layer "B.Cu") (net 2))
 (segment (start 152.042176 121.330389) (end 151.603108 121.330389) (width 0.16) (layer "B.Cu") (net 2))
 (segment (start 150.142642 102.102889) (end 151.692642 102.102889) (width 0.16) (layer "B.Cu") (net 2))
 (segment (start 145.527642 122.310389) (end 145.457642 122.240389) (width 0.16) (layer "B.Cu") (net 2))
 (segment (start 148.485142 100.320389) (end 148.485142 102.000389) (width 0.16) (layer "B.Cu") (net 2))
 (segment (start 148.887642 122.310389) (end 145.527642 122.310389) (width 0.16) (layer "B.Cu") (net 2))
 (segment (start 148.485142 100.320389) (end 148.485142 100.302889) (width 0.16) (layer "B.Cu") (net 2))
 (segment (start 148.587642 102.102889) (end 148.505142 102.020389) (width 0.16) (layer "B.Cu") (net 2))
 (segment (start 149.887642 91.622889) (end 149.887642 97.435389) (width 0.16) (layer "B.Cu") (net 2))
 (segment (start 147.202642 104.100389) (end 147.202642 103.322889) (width 0.16) (layer "B.Cu") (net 2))
 (segment (start 147.202642 103.322889) (end 148.505142 102.020389) (width 0.16) (layer "B.Cu") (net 2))
 (segment (start 148.485142 102.000389) (end 148.505142 102.020389) (width 0.16) (layer "B.Cu") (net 2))
 (segment (start 148.485142 100.302889) (end 148.712642 100.075389) (width 0.16) (layer "B.Cu") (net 2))
 (segment (start 152.352642 125.150389) (end 152.352642 121.640855) (width 0.16) (layer "B.Cu") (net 2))
 (segment (start 148.957642 105.855389) (end 147.202642 104.100389) (width 0.16) (layer "B.Cu") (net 2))
 (segment (start 148.957642 122.240389) (end 148.887642 122.310389) (width 0.16) (layer "B.Cu") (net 2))
 (segment (start 145.457642 122.240389) (end 145.457642 121.580389) (width 0.16) (layer "B.Cu") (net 2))
 (segment (start 149.687642 122.310389) (end 148.957642 121.580389) (width 0.16) (layer "B.Cu") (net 2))
 (segment (start 145.172642 100.297889) (end 146.737642 100.297889) (width 0.16) (layer "B.Cu") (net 6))
 (segment (start 146.737642 100.297889) (end 146.760142 100.320389) (width 0.16) (layer "B.Cu") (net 6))
 (segment (start 145.172642 94.825237) (end 146.957642 93.040237) (width 0.16) (layer "B.Cu") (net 6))
 (segment (start 145.172642 100.297889) (end 145.172642 94.825237) (width 0.16) (layer "B.Cu") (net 6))
 (segment (start 146.957642 93.040237) (end 146.957642 92.352889) (width 0.16) (layer "B.Cu") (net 6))
 (segment (start 149.457642 94.017889) (end 148.535142 94.940389) (width 0.16) (layer "B.Cu") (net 7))
 (segment (start 148.535142 96.432889) (end 148.712642 96.610389) (width 0.16) (layer "B.Cu") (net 7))
 (segment (start 149.457642 92.352889) (end 149.457642 94.017889) (width 0.16) (layer "B.Cu") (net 7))
 (segment (start 148.535142 94.940389) (end 148.535142 96.432889) (width 0.16) (layer "B.Cu") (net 7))
 (segment (start 146.809624 93.697371) (end 146.809624 94.939871) (width 0.16) (layer "B.Cu") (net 4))
 (segment (start 146.682642 95.067889) (end 146.810142 94.940389) (width 0.16) (layer "B.Cu") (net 4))
 (segment (start 147.457642 93.049353) (end 146.809624 93.697371) (width 0.16) (layer "B.Cu") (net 4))
 (segment (start 146.809624 94.939871) (end 146.810142 94.940389) (width 0.16) (layer "B.Cu") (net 4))
 (segment (start 146.682642 96.630389) (end 146.682642 95.067889) (width 0.16) (layer "B.Cu") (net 4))
 (segment (start 147.457642 92.352889) (end 147.457642 93.049353) (width 0.16) (layer "B.Cu") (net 4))
 (segment (start 147.662642 93.560389) (end 147.662642 97.650389) (width 0.16) (layer "B.Cu") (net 5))
 (segment (start 147.577642 101.222889) (end 147.577642 99.525389) (width 0.16) (layer "B.Cu") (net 5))
 (segment (start 146.677642 102.122889) (end 146.780142 102.020389) (width 0.16) (layer "B.Cu") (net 5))
 (segment (start 148.457642 105.975389) (end 146.780142 104.297889) (width 0.16) (layer "B.Cu") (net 5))
 (segment (start 148.457642 121.580389) (end 148.457642 105.975389) (width 0.16) (layer "B.Cu") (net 5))
 (segment (start 146.780142 102.020389) (end 147.577642 101.222889) (width 0.16) (layer "B.Cu") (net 5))
 (segment (start 147.577642 99.525389) (end 146.682642 98.630389) (width 0.16) (layer "B.Cu") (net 5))
 (segment (start 145.172642 102.122889) (end 146.677642 102.122889) (width 0.16) (layer "B.Cu") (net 5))
 (segment (start 147.957642 93.265389) (end 147.662642 93.560389) (width 0.16) (layer "B.Cu") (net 5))
 (segment (start 147.957642 92.352889) (end 147.957642 93.265389) (width 0.16) (layer "B.Cu") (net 5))
 (segment (start 146.780142 104.297889) (end 146.780142 102.020389) (width 0.16) (layer "B.Cu") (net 5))
 (segment (start 147.662642 97.650389) (end 146.682642 98.630389) (width 0.16) (layer "B.Cu") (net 5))
 (segment (start 143.697642 99.528719) (end 143.697642 103.465389) (width 0.16) (layer "B.Cu") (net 10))
 (segment (start 143.702642 99.523719) (end 143.697642 99.528719) (width 0.16) (layer "B.Cu") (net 10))
 (segment (start 144.957642 92.352889) (end 144.957642 92.956273) (width 0.16) (layer "B.Cu") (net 10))
 (segment (start 143.702642 94.211273) (end 143.702642 99.523719) (width 0.16) (layer "B.Cu") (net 10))
 (segment (start 143.697642 103.465389) (end 146.957642 106.725389) (width 0.16) (layer "B.Cu") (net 10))
 (segment (start 144.957642 92.956273) (end 143.702642 94.211273) (width 0.16) (layer "B.Cu") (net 10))
 (segment (start 146.957642 106.725389) (end 146.957642 121.580389) (width 0.16) (layer "B.Cu") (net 10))
 (segment (start 145.457642 92.352889) (end 145.457642 92.965389) (width 0.16) (layer "B.Cu") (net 9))
 (segment (start 144.057642 102.935389) (end 147.457642 106.335389) (width 0.16) (layer "B.Cu") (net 9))
 (segment (start 144.062642 94.360389) (end 144.062642 99.672836) (width 0.16) (layer "B.Cu") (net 9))
 (segment (start 144.057642 99.677836) (end 144.057642 102.935389) (width 0.16) (layer "B.Cu") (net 9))
 (segment (start 147.457642 106.335389) (end 147.457642 121.580389) (width 0.16) (layer "B.Cu") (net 9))
 (segment (start 145.457642 92.965389) (end 144.062642 94.360389) (width 0.16) (layer "B.Cu") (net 9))
 (segment (start 144.062642 99.672836) (end 144.057642 99.677836) (width 0.16) (layer "B.Cu") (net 9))
 (segment (start 145.957642 92.352889) (end 145.957642 93.022005) (width 0.16) (layer "B.Cu") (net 8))
 (segment (start 147.957642 106.133825) (end 147.957642 121.580389) (width 0.16) (layer "B.Cu") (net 8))
 (segment (start 144.422642 99.821953) (end 144.417642 99.826953) (width 0.16) (layer "B.Cu") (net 8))
 (segment (start 144.417642 99.826953) (end 144.417642 102.593825) (width 0.16) (layer "B.Cu") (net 8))
 (segment (start 145.957642 93.022005) (end 144.422642 94.557005) (width 0.16) (layer "B.Cu") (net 8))
 (segment (start 144.422642 94.557005) (end 144.422642 99.821953) (width 0.16) (layer "B.Cu") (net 8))
 (segment (start 144.417642 102.593825) (end 147.957642 106.133825) (width 0.16) (layer "B.Cu") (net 8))
 (segment (start 148.457642 91.675389) (end 148.457642 92.352889) (width 0.16) (layer "B.Cu") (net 11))
 (segment (start 150.036759 91.262889) (end 148.870142 91.262889) (width 0.16) (layer "B.Cu") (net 11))
 (segment (start 150.142642 100.277889) (end 150.247642 100.172889) (width 0.16) (layer "B.Cu") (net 11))
 (segment (start 150.247642 91.473772) (end 150.036759 91.262889) (width 0.16) (layer "B.Cu") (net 11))
 (segment (start 148.870142 91.262889) (end 148.457642 91.675389) (width 0.16) (layer "B.Cu") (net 11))
 (segment (start 150.247642 100.172889) (end 150.247642 91.473772) (width 0.16) (layer "B.Cu") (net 11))
 (segment (start 146.457642 92.352889) (end 146.457642 91.692889) (width 0.16) (layer "B.Cu") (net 12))
 (segment (start 148.001026 91.622889) (end 148.721026 90.902889) (width 0.16) (layer "B.Cu") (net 12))
 (segment (start 148.721026 90.902889) (end 150.195142 90.902889) (width 0.16) (layer "B.Cu") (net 12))
 (segment (start 146.457642 91.692889) (end 146.527642 91.622889) (width 0.16) (layer "B.Cu") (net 12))
 (segment (start 150.195142 90.902889) (end 150.607642 91.315389) (width 0.16) (layer "B.Cu") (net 12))
 (segment (start 150.607642 99.192889) (end 151.692642 100.277889) (width 0.16) (layer "B.Cu") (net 12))
 (segment (start 146.527642 91.622889) (end 148.001026 91.622889) (width 0.16) (layer "B.Cu") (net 12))
 (segment (start 150.607642 91.315389) (end 150.607642 99.192889) (width 0.16) (layer "B.Cu") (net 12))
 (segment (start 139.570142 121.860389) (end 142.582642 121.860389) (width 0.16) (layer "F.Cu") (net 3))
 (segment (start 142.582642 121.860389) (end 145.570142 121.860389) (width 0.16) (layer "F.Cu") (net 3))
 (via (at 142.582642 121.860389) (size 0.5) (drill 0.3) (layers "F.Cu" "B.Cu") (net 3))
 (segment (start 146.457642 120.911273) (end 146.006758 120.460389) (width 0.16) (layer "B.Cu") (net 3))
 (segment (start 143.462642 121.860389) (end 142.582642 121.860389) (width 0.16) (layer "B.Cu") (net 3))
 (segment (start 144.862642 120.460389) (end 143.462642 121.860389) (width 0.16) (layer "B.Cu") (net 3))
 (segment (start 146.006758 120.460389) (end 144.862642 120.460389) (width 0.16) (layer "B.Cu") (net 3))
 (segment (start 146.457642 121.580389) (end 146.457642 120.911273) (width 0.16) (layer "B.Cu") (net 3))
 (segment (start 151.822642 121.860389) (end 154.845142 121.860389) (width 0.16) (layer "F.Cu") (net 1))
 (segment (start 148.845142 121.860389) (end 151.822642 121.860389) (width 0.16) (layer "F.Cu") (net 1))
 (via (at 151.822642 121.860389) (size 0.5) (drill 0.3) (layers "F.Cu" "B.Cu") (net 1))
 (segment (start 144.392642 122.190389) (end 144.872642 122.670389) (width 0.16) (layer "B.Cu") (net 1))
 (segment (start 145.857642 120.820389) (end 145.011758 120.820389) (width 0.16) (layer "B.Cu") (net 1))
 (segment (start 145.957642 120.920389) (end 145.857642 120.820389) (width 0.16) (layer "B.Cu") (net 1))
 (segment (start 145.011758 120.820389) (end 144.392642 121.439505) (width 0.16) (layer "B.Cu") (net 1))
 (segment (start 151.012642 122.670389) (end 151.822642 121.860389) (width 0.16) (layer "B.Cu") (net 1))
 (segment (start 145.957642 121.580389) (end 145.957642 120.920389) (width 0.16) (layer "B.Cu") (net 1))
 (segment (start 144.872642 122.670389) (end 151.012642 122.670389) (width 0.16) (layer "B.Cu") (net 1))
 (segment (start 144.392642 121.439505) (end 144.392642 122.190389) (width 0.16) (layer "B.Cu") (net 1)))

